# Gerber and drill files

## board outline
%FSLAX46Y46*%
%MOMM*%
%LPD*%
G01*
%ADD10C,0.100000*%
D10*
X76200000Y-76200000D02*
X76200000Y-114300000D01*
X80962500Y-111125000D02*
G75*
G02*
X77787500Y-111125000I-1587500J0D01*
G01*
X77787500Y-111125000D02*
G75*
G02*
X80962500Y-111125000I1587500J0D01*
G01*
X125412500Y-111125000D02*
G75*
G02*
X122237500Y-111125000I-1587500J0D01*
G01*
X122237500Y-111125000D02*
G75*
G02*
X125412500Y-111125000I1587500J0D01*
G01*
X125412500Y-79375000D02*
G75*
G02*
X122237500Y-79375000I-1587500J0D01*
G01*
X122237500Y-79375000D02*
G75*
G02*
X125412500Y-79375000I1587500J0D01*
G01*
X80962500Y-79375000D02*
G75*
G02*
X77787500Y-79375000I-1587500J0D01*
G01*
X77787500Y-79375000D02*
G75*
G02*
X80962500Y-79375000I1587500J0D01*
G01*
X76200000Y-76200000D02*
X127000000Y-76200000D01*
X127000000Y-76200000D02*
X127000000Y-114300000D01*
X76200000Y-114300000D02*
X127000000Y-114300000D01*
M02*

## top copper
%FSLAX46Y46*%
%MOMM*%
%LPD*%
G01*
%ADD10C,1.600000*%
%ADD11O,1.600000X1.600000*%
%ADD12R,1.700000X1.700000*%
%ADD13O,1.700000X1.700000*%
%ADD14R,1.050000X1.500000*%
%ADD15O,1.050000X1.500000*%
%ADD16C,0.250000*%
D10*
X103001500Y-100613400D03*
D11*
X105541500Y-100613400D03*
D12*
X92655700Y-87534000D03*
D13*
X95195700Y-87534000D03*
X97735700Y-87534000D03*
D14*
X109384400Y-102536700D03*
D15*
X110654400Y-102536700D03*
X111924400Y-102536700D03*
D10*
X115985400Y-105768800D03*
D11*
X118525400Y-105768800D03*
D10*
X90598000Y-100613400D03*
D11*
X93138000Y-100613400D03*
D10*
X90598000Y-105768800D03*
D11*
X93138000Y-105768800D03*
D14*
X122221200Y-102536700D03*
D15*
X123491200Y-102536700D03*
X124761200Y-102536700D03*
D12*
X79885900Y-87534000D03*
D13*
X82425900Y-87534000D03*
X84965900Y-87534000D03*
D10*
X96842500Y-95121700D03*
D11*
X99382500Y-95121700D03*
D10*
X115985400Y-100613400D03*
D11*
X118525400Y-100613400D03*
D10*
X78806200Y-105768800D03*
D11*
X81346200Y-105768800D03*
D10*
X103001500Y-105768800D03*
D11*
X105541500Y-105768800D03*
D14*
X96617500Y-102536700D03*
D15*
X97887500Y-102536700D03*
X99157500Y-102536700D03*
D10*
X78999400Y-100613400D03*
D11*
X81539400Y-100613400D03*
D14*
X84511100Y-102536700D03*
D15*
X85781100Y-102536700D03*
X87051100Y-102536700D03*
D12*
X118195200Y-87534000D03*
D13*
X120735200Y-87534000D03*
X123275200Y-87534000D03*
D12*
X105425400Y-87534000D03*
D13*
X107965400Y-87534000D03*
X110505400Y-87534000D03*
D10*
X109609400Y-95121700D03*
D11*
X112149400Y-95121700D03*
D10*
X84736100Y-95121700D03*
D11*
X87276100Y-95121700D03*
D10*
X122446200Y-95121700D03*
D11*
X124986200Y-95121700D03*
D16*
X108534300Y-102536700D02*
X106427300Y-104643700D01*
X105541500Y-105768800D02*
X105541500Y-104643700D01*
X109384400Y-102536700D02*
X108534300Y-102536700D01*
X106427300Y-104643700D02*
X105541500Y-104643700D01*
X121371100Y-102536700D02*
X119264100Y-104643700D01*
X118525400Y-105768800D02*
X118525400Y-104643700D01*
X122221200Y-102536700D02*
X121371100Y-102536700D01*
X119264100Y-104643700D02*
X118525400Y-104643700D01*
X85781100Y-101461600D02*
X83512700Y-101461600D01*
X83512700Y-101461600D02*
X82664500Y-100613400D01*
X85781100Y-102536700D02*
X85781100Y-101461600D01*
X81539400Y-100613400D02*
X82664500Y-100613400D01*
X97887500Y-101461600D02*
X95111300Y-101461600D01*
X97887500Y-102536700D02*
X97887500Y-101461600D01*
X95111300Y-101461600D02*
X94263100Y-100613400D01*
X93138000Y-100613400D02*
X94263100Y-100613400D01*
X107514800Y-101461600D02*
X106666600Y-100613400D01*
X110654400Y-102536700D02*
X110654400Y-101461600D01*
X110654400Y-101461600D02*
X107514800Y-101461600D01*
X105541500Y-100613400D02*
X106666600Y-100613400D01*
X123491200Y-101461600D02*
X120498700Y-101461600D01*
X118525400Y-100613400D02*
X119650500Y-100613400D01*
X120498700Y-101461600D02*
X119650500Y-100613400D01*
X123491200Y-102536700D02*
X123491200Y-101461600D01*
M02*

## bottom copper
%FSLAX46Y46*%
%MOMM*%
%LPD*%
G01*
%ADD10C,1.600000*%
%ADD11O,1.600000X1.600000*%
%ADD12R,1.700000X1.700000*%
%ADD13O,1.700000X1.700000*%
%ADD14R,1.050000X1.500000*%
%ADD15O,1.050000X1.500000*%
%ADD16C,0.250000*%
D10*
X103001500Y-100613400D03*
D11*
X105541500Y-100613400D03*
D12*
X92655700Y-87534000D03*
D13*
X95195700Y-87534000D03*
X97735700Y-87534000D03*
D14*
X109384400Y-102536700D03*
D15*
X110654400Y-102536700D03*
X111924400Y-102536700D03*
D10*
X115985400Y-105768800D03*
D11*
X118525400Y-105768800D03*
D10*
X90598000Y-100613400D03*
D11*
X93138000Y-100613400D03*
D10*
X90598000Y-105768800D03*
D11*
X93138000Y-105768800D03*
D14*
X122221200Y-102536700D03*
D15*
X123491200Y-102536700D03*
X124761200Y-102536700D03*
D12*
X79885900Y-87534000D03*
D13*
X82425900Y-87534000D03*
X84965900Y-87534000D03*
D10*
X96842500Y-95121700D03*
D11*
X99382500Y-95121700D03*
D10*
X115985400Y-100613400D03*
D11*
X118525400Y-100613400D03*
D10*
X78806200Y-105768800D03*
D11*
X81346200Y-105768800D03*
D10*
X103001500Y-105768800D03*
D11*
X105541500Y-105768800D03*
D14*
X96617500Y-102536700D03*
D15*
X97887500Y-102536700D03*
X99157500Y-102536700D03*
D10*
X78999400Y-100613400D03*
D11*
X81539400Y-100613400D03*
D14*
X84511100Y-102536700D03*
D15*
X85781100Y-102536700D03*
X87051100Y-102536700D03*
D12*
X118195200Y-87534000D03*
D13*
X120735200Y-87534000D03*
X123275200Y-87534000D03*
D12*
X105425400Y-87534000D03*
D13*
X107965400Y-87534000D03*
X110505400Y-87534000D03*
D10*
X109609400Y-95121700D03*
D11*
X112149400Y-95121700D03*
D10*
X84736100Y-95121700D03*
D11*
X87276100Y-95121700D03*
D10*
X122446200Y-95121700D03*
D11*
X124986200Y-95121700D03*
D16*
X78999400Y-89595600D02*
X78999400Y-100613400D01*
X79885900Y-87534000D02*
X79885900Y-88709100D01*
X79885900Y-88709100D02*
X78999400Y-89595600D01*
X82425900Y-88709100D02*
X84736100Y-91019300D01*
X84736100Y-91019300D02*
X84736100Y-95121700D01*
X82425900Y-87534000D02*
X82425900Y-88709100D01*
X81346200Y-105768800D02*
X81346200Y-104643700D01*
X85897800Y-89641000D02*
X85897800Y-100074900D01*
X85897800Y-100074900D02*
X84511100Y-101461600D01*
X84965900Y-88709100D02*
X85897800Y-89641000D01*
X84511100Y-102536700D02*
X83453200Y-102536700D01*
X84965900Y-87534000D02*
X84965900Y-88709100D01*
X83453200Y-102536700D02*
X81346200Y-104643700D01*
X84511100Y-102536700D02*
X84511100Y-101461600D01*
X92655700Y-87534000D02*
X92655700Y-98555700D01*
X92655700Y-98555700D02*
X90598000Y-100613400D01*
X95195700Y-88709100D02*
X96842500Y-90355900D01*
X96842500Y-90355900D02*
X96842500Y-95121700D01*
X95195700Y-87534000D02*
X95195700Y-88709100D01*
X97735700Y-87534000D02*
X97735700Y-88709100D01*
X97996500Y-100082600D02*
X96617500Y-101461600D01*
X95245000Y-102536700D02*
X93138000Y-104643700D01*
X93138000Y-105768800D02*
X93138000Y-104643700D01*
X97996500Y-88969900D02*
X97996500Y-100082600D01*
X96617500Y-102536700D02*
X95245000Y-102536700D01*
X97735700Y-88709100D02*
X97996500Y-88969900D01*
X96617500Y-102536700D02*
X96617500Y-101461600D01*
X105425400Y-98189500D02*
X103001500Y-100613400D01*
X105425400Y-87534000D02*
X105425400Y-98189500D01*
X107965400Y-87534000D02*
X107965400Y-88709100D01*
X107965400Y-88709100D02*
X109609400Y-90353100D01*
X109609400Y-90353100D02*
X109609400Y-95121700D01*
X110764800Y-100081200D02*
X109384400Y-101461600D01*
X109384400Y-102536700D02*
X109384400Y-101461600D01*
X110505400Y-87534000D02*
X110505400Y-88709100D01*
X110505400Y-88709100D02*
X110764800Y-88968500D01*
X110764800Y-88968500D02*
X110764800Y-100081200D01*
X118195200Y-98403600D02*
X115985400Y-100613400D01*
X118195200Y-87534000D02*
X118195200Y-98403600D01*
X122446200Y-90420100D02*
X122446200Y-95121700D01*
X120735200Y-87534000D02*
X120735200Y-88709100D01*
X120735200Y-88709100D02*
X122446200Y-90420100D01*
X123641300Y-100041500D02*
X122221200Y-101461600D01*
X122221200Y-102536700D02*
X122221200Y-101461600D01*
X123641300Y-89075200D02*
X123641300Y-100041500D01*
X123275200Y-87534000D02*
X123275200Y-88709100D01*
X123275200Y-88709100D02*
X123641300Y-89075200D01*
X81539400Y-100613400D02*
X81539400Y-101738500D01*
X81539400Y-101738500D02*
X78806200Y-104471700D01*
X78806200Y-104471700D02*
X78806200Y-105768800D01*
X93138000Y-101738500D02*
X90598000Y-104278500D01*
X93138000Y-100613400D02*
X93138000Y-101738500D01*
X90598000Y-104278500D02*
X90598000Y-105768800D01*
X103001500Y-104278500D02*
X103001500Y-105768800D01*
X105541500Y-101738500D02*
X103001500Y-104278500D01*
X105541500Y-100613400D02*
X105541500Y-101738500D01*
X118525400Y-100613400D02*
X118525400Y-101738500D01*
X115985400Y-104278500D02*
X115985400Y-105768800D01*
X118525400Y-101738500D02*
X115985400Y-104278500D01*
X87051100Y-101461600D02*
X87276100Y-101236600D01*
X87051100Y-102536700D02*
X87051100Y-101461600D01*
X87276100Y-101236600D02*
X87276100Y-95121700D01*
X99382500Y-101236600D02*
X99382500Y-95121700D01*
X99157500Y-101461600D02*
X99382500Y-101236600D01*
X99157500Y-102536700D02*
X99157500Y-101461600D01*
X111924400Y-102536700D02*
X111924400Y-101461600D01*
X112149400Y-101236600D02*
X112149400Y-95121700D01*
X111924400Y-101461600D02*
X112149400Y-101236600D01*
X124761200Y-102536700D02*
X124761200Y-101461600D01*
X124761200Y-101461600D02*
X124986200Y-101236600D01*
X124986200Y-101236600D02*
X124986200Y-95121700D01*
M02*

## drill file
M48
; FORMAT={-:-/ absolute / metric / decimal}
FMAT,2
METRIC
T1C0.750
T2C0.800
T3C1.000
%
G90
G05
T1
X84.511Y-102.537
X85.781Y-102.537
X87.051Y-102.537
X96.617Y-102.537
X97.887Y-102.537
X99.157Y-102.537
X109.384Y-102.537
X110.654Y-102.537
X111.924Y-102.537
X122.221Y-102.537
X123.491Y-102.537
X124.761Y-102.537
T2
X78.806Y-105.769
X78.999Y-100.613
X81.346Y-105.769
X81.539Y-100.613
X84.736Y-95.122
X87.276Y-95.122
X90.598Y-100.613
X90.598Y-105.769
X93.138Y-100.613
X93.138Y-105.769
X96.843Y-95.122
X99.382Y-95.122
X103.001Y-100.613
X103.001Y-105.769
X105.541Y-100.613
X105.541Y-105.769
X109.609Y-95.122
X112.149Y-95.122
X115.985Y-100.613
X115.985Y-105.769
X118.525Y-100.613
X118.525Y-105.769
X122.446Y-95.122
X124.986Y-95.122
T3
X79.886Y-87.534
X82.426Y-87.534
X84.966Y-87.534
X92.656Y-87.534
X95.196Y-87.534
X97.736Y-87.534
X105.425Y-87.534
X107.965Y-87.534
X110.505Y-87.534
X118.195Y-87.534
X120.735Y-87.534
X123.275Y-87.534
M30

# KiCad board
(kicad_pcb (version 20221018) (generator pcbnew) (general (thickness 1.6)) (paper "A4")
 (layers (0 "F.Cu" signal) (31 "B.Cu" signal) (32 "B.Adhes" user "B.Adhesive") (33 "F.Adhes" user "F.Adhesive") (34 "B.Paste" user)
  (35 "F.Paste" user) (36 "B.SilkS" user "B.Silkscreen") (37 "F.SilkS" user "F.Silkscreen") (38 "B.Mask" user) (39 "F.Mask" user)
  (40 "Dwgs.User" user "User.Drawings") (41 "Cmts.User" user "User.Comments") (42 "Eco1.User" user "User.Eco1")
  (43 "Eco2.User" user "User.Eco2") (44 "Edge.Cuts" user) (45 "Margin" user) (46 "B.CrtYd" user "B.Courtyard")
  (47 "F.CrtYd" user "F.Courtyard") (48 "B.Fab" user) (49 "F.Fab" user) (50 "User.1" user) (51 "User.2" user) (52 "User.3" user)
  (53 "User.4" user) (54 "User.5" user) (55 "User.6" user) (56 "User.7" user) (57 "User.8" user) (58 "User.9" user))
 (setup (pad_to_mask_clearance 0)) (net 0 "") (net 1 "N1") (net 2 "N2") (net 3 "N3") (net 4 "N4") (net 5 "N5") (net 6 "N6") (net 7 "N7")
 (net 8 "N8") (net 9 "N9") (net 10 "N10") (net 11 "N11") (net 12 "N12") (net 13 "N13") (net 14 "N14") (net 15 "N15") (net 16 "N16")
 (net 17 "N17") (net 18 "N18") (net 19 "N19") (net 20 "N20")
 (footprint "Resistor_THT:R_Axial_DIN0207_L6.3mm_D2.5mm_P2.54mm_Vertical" (layer "F.Cu") (at 103.0015 100.6134)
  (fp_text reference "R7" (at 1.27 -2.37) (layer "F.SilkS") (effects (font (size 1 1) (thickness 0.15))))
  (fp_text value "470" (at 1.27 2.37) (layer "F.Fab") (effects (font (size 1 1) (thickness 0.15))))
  (pad "1" thru_hole circle (at 0 0) (size 1.6 1.6) (drill 0.8) (layers "*.Cu" "*.Mask") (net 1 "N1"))
  (pad "2" thru_hole oval (at 2.54 0) (size 1.6 1.6) (drill 0.8) (layers "*.Cu" "*.Mask") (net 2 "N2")))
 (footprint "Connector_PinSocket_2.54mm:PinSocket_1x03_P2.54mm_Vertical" (layer "F.Cu") (at 92.6557 87.534 90)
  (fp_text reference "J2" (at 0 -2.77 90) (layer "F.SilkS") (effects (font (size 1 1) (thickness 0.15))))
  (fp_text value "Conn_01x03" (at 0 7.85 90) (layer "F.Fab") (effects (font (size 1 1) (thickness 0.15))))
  (pad "1" thru_hole rect (at 0 0 90) (size 1.7 1.7) (drill 1) (layers "*.Cu" "*.Mask") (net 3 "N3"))
  (pad "2" thru_hole oval (at 0 2.54 90) (size 1.7 1.7) (drill 1) (layers "*.Cu" "*.Mask") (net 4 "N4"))
  (pad "3" thru_hole oval (at 0 5.08 90) (size 1.7 1.7) (drill 1) (layers "*.Cu" "*.Mask") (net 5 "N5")))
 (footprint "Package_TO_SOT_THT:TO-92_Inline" (layer "F.Cu") (at 109.3844 102.5367)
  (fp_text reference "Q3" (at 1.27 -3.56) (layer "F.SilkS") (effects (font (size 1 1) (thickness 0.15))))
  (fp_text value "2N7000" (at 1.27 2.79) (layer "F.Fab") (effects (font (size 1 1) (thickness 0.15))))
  (pad "1" thru_hole rect (at 0 0) (size 1.05 1.5) (drill 0.75) (layers "*.Cu" "*.Mask") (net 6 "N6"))
  (pad "2" thru_hole oval (at 1.27 0) (size 1.05 1.5) (drill 0.75) (layers "*.Cu" "*.Mask") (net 2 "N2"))
  (pad "3" thru_hole oval (at 2.54 0) (size 1.05 1.5) (drill 0.75) (layers "*.Cu" "*.Mask") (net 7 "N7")))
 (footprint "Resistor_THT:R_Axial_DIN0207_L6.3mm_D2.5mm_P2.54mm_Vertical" (layer "F.Cu") (at 115.9854 105.7688)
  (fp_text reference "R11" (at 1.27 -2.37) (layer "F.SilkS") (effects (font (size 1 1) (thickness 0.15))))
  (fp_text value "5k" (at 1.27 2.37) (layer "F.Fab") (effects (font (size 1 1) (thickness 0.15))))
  (pad "1" thru_hole circle (at 0 0) (size 1.6 1.6) (drill 0.8) (layers "*.Cu" "*.Mask") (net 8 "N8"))
  (pad "2" thru_hole oval (at 2.54 0) (size 1.6 1.6) (drill 0.8) (layers "*.Cu" "*.Mask") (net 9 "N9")))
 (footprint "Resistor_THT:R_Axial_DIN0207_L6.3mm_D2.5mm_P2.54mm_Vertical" (layer "F.Cu") (at 90.598 100.6134)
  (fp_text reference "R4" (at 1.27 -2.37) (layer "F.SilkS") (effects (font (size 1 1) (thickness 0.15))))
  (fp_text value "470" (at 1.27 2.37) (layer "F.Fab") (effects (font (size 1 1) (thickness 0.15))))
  (pad "1" thru_hole circle (at 0 0) (size 1.6 1.6) (drill 0.8) (layers "*.Cu" "*.Mask") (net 3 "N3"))
  (pad "2" thru_hole oval (at 2.54 0) (size 1.6 1.6) (drill 0.8) (layers "*.Cu" "*.Mask") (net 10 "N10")))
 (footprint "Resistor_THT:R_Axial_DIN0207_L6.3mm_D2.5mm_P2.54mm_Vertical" (layer "F.Cu") (at 90.598 105.7688)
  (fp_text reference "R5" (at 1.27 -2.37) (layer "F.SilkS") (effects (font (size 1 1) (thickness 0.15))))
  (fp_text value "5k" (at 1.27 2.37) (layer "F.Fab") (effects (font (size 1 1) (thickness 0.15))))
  (pad "1" thru_hole circle (at 0 0) (size 1.6 1.6) (drill 0.8) (layers "*.Cu" "*.Mask") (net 10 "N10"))
  (pad "2" thru_hole oval (at 2.54 0) (size 1.6 1.6) (drill 0.8) (layers "*.Cu" "*.Mask") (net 5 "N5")))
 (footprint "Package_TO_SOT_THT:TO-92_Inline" (layer "F.Cu") (at 122.2212 102.5367)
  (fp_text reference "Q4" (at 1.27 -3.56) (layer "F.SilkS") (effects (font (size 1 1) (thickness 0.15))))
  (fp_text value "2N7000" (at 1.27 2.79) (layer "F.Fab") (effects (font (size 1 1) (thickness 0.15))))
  (pad "1" thru_hole rect (at 0 0) (size 1.05 1.5) (drill 0.75) (layers "*.Cu" "*.Mask") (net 9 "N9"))
  (pad "2" thru_hole oval (at 1.27 0) (size 1.05 1.5) (drill 0.75) (layers "*.Cu" "*.Mask") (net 8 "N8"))
  (pad "3" thru_hole oval (at 2.54 0) (size 1.05 1.5) (drill 0.75) (layers "*.Cu" "*.Mask") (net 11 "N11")))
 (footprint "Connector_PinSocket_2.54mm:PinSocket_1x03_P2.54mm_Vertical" (layer "F.Cu") (at 79.8859 87.534 90)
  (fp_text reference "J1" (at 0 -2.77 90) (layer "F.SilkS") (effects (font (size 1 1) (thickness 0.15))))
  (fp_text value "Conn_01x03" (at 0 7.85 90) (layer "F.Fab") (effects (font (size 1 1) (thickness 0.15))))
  (pad "1" thru_hole rect (at 0 0 90) (size 1.7 1.7) (drill 1) (layers "*.Cu" "*.Mask") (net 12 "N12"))
  (pad "2" thru_hole oval (at 0 2.54 90) (size 1.7 1.7) (drill 1) (layers "*.Cu" "*.Mask") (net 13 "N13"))
  (pad "3" thru_hole oval (at 0 5.08 90) (size 1.7 1.7) (drill 1) (layers "*.Cu" "*.Mask") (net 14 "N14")))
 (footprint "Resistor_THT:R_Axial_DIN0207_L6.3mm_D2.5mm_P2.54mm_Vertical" (layer "F.Cu") (at 96.8425 95.1217)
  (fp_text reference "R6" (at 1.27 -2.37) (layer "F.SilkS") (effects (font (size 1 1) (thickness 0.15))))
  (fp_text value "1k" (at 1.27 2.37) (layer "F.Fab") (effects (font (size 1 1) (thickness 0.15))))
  (pad "1" thru_hole circle (at 0 0) (size 1.6 1.6) (drill 0.8) (layers "*.Cu" "*.Mask") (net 4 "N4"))
  (pad "2" thru_hole oval (at 2.54 0) (size 1.6 1.6) (drill 0.8) (layers "*.Cu" "*.Mask") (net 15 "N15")))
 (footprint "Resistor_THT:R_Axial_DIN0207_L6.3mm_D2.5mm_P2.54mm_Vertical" (layer "F.Cu") (at 115.9854 100.6134)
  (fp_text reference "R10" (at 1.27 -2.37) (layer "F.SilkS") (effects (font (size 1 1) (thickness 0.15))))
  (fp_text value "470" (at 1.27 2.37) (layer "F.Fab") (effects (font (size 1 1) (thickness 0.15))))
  (pad "1" thru_hole circle (at 0 0) (size 1.6 1.6) (drill 0.8) (layers "*.Cu" "*.Mask") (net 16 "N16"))
  (pad "2" thru_hole oval (at 2.54 0) (size 1.6 1.6) (drill 0.8) (layers "*.Cu" "*.Mask") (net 8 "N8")))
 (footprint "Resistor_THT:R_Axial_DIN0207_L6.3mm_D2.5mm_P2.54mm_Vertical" (layer "F.Cu") (at 78.8062 105.7688)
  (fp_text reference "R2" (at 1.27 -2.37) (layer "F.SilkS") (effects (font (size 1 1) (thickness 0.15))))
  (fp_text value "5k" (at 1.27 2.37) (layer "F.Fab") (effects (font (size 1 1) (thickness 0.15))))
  (pad "1" thru_hole circle (at 0 0) (size 1.6 1.6) (drill 0.8) (layers "*.Cu" "*.Mask") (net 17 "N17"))
  (pad "2" thru_hole oval (at 2.54 0) (size 1.6 1.6) (drill 0.8) (layers "*.Cu" "*.Mask") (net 14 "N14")))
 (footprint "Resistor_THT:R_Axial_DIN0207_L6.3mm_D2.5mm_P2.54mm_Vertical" (layer "F.Cu") (at 103.0015 105.7688)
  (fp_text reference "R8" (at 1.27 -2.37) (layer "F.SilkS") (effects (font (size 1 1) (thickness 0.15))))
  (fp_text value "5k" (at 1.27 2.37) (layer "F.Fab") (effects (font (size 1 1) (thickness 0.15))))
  (pad "1" thru_hole circle (at 0 0) (size 1.6 1.6) (drill 0.8) (layers "*.Cu" "*.Mask") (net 2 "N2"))
  (pad "2" thru_hole oval (at 2.54 0) (size 1.6 1.6) (drill 0.8) (layers "*.Cu" "*.Mask") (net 6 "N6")))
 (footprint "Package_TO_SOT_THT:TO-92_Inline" (layer "F.Cu") (at 96.6175 102.5367)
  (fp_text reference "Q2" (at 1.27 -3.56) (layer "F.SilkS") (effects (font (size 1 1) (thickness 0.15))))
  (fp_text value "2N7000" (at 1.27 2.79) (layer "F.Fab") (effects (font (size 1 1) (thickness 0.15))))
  (pad "1" thru_hole rect (at 0 0) (size 1.05 1.5) (drill 0.75) (layers "*.Cu" "*.Mask") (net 5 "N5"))
  (pad "2" thru_hole oval (at 1.27 0) (size 1.05 1.5) (drill 0.75) (layers "*.Cu" "*.Mask") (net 10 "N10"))
  (pad "3" thru_hole oval (at 2.54 0) (size 1.05 1.5) (drill 0.75) (layers "*.Cu" "*.Mask") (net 15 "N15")))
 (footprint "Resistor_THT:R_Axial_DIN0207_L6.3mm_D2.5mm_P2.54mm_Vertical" (layer "F.Cu") (at 78.9994 100.6134)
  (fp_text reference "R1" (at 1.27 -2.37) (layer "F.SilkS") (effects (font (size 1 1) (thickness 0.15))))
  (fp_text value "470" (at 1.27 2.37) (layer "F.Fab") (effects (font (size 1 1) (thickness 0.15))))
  (pad "1" thru_hole circle (at 0 0) (size 1.6 1.6) (drill 0.8) (layers "*.Cu" "*.Mask") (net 12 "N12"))
  (pad "2" thru_hole oval (at 2.54 0) (size 1.6 1.6) (drill 0.8) (layers "*.Cu" "*.Mask") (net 17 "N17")))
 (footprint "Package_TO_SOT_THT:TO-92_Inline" (layer "F.Cu") (at 84.5111 102.5367)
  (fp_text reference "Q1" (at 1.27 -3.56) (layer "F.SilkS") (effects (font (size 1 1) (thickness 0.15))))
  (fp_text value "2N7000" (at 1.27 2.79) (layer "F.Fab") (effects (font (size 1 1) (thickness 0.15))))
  (pad "1" thru_hole rect (at 0 0) (size 1.05 1.5) (drill 0.75) (layers "*.Cu" "*.Mask") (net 14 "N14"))
  (pad "2" thru_hole oval (at 1.27 0) (size 1.05 1.5) (drill 0.75) (layers "*.Cu" "*.Mask") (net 17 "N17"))
  (pad "3" thru_hole oval (at 2.54 0) (size 1.05 1.5) (drill 0.75) (layers "*.Cu" "*.Mask") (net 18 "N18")))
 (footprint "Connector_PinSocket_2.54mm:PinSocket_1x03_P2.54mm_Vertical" (layer "F.Cu") (at 118.1952 87.534 90)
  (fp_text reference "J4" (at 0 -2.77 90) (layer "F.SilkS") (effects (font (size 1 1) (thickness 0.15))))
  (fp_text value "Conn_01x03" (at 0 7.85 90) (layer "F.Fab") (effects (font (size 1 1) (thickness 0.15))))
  (pad "1" thru_hole rect (at 0 0 90) (size 1.7 1.7) (drill 1) (layers "*.Cu" "*.Mask") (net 16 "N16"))
  (pad "2" thru_hole oval (at 0 2.54 90) (size 1.7 1.7) (drill 1) (layers "*.Cu" "*.Mask") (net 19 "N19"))
  (pad "3" thru_hole oval (at 0 5.08 90) (size 1.7 1.7) (drill 1) (layers "*.Cu" "*.Mask") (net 9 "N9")))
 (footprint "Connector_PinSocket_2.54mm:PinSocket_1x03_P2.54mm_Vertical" (layer "F.Cu") (at 105.4254 87.534 90)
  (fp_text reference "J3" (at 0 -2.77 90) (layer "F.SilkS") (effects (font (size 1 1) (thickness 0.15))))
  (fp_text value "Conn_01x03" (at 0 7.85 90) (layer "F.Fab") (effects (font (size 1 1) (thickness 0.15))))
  (pad "1" thru_hole rect (at 0 0 90) (size 1.7 1.7) (drill 1) (layers "*.Cu" "*.Mask") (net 1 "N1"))
  (pad "2" thru_hole oval (at 0 2.54 90) (size 1.7 1.7) (drill 1) (layers "*.Cu" "*.Mask") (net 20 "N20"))
  (pad "3" thru_hole oval (at 0 5.08 90) (size 1.7 1.7) (drill 1) (layers "*.Cu" "*.Mask") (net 6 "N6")))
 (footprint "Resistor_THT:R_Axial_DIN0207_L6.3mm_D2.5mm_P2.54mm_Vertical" (layer "F.Cu") (at 109.6094 95.1217)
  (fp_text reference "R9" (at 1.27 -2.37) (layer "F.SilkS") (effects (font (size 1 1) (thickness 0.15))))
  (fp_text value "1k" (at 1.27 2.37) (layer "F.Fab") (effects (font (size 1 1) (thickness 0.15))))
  (pad "1" thru_hole circle (at 0 0) (size 1.6 1.6) (drill 0.8) (layers "*.Cu" "*.Mask") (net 20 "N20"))
  (pad "2" thru_hole oval (at 2.54 0) (size 1.6 1.6) (drill 0.8) (layers "*.Cu" "*.Mask") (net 7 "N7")))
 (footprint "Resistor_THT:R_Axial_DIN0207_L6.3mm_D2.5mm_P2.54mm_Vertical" (layer "F.Cu") (at 84.7361 95.1217)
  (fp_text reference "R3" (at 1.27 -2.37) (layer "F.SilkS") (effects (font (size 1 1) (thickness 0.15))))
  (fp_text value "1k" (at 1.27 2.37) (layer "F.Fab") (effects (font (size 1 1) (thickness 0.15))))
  (pad "1" thru_hole circle (at 0 0) (size 1.6 1.6) (drill 0.8) (layers "*.Cu" "*.Mask") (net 13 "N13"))
  (pad "2" thru_hole oval (at 2.54 0) (size 1.6 1.6) (drill 0.8) (layers "*.Cu" "*.Mask") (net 18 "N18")))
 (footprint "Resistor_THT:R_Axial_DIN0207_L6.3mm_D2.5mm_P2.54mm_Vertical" (layer "F.Cu") (at 122.4462 95.1217)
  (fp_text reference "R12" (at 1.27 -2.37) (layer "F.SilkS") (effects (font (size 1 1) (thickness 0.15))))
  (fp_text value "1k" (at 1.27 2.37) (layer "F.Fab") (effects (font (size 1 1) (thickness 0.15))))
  (pad "1" thru_hole circle (at 0 0) (size 1.6 1.6) (drill 0.8) (layers "*.Cu" "*.Mask") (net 19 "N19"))
  (pad "2" thru_hole oval (at 2.54 0) (size 1.6 1.6) (drill 0.8) (layers "*.Cu" "*.Mask") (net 11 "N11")))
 (gr_line (start 76.2 76.2) (end 76.2 114.3) (stroke (width 0.1) (type default)) (layer "Edge.Cuts"))
 (gr_circle (center 79.375 111.125) (end 80.9625 111.125) (stroke (width 0.1) (type default)) (fill none) (layer "Edge.Cuts"))
 (gr_circle (center 123.825 111.125) (end 125.4125 111.125) (stroke (width 0.1) (type default)) (fill none) (layer "Edge.Cuts"))
 (gr_circle (center 123.825 79.375) (end 125.4125 79.375) (stroke (width 0.1) (type default)) (fill none) (layer "Edge.Cuts"))
 (gr_circle (center 79.375 79.375) (end 80.9625 79.375) (stroke (width 0.1) (type default)) (fill none) (layer "Edge.Cuts"))
 (gr_line (start 76.2 76.2) (end 127 76.2) (stroke (width 0.1) (type default)) (layer "Edge.Cuts"))
 (gr_line (start 127 76.2) (end 127 114.3) (stroke (width 0.1) (type default)) (layer "Edge.Cuts"))
 (gr_line (start 76.2 114.3) (end 127 114.3) (stroke (width 0.1) (type default)) (layer "Edge.Cuts"))
 (segment (start 78.9994 89.5956) (end 78.9994 100.6134) (width 0.25) (layer "B.Cu") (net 12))
 (segment (start 79.8859 87.534) (end 79.8859 88.7091) (width 0.25) (layer "B.Cu") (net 12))
 (segment (start 79.8859 88.7091) (end 78.9994 89.5956) (width 0.25) (layer "B.Cu") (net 12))
 (segment (start 82.4259 88.7091) (end 84.7361 91.0193) (width 0.25) (layer "B.Cu") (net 13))
 (segment (start 84.7361 91.0193) (end 84.7361 95.1217) (width 0.25) (layer "B.Cu") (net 13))
 (segment (start 82.4259 87.534) (end 82.4259 88.7091) (width 0.25) (layer "B.Cu") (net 13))
 (segment (start 81.3462 105.7688) (end 81.3462 104.6437) (width 0.25) (layer "B.Cu") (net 14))
 (segment (start 85.8978 89.641) (end 85.8978 100.0749) (width 0.25) (layer "B.Cu") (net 14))
 (segment (start 85.8978 100.0749) (end 84.5111 101.4616) (width 0.25) (layer "B.Cu") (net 14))
 (segment (start 84.9659 88.7091) (end 85.8978 89.641) (width 0.25) (layer "B.Cu") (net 14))
 (segment (start 84.5111 102.5367) (end 83.4532 102.5367) (width 0.25) (layer "B.Cu") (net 14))
 (segment (start 84.9659 87.534) (end 84.9659 88.7091) (width 0.25) (layer "B.Cu") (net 14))
 (segment (start 83.4532 102.5367) (end 81.3462 104.6437) (width 0.25) (layer "B.Cu") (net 14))
 (segment (start 84.5111 102.5367) (end 84.5111 101.4616) (width 0.25) (layer "B.Cu") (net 14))
 (segment (start 92.6557 87.534) (end 92.6557 98.5557) (width 0.25) (layer "B.Cu") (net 3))
 (segment (start 92.6557 98.5557) (end 90.598 100.6134) (width 0.25) (layer "B.Cu") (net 3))
 (segment (start 95.1957 88.7091) (end 96.8425 90.3559) (width 0.25) (layer "B.Cu") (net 4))
 (segment (start 96.8425 90.3559) (end 96.8425 95.1217) (width 0.25) (layer "B.Cu") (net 4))
 (segment (start 95.1957 87.534) (end 95.1957 88.7091) (width 0.25) (layer "B.Cu") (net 4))
 (segment (start 97.7357 87.534) (end 97.7357 88.7091) (width 0.25) (layer "B.Cu") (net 5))
 (segment (start 97.9965 100.0826) (end 96.6175 101.4616) (width 0.25) (layer "B.Cu") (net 5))
 (segment (start 95.245 102.5367) (end 93.138 104.6437) (width 0.25) (layer "B.Cu") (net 5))
 (segment (start 93.138 105.7688) (end 93.138 104.6437) (width 0.25) (layer "B.Cu") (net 5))
 (segment (start 97.9965 88.9699) (end 97.9965 100.0826) (width 0.25) (layer "B.Cu") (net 5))
 (segment (start 96.6175 102.5367) (end 95.245 102.5367) (width 0.25) (layer "B.Cu") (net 5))
 (segment (start 97.7357 88.7091) (end 97.9965 88.9699) (width 0.25) (layer "B.Cu") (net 5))
 (segment (start 96.6175 102.5367) (end 96.6175 101.4616) (width 0.25) (layer "B.Cu") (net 5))
 (segment (start 105.4254 98.1895) (end 103.0015 100.6134) (width 0.25) (layer "B.Cu") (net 1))
 (segment (start 105.4254 87.534) (end 105.4254 98.1895) (width 0.25) (layer "B.Cu") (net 1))
 (segment (start 107.9654 87.534) (end 107.9654 88.7091) (width 0.25) (layer "B.Cu") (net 20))
 (segment (start 107.9654 88.7091) (end 109.6094 90.3531) (width 0.25) (layer "B.Cu") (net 20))
 (segment (start 109.6094 90.3531) (end 109.6094 95.1217) (width 0.25) (layer "B.Cu") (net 20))
 (segment (start 108.5343 102.5367) (end 106.4273 104.6437) (width 0.25) (layer "F.Cu") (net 6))
 (segment (start 105.5415 105.7688) (end 105.5415 104.6437) (width 0.25) (layer "F.Cu") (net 6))
 (segment (start 109.3844 102.5367) (end 108.5343 102.5367) (width 0.25) (layer "F.Cu") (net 6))
 (segment (start 106.4273 104.6437) (end 105.5415 104.6437) (width 0.25) (layer "F.Cu") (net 6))
 (segment (start 110.7648 100.0812) (end 109.3844 101.4616) (width 0.25) (layer "B.Cu") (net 6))
 (segment (start 109.3844 102.5367) (end 109.3844 101.4616) (width 0.25) (layer "B.Cu") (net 6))
 (segment (start 110.5054 87.534) (end 110.5054 88.7091) (width 0.25) (layer "B.Cu") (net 6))
 (segment (start 110.5054 88.7091) (end 110.7648 88.9685) (width 0.25) (layer "B.Cu") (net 6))
 (segment (start 110.7648 88.9685) (end 110.7648 100.0812) (width 0.25) (layer "B.Cu") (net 6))
 (segment (start 118.1952 98.4036) (end 115.9854 100.6134) (width 0.25) (layer "B.Cu") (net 16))
 (segment (start 118.1952 87.534) (end 118.1952 98.4036) (width 0.25) (layer "B.Cu") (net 16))
 (segment (start 122.4462 90.4201) (end 122.4462 95.1217) (width 0.25) (layer "B.Cu") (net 19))
 (segment (start 120.7352 87.534) (end 120.7352 88.7091) (width 0.25) (layer "B.Cu") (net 19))
 (segment (start 120.7352 88.7091) (end 122.4462 90.4201) (width 0.25) (layer "B.Cu") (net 19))
 (segment (start 121.3711 102.5367) (end 119.2641 104.6437) (width 0.25) (layer "F.Cu") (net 9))
 (segment (start 118.5254 105.7688) (end 118.5254 104.6437) (width 0.25) (layer "F.Cu") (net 9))
 (segment (start 122.2212 102.5367) (end 121.3711 102.5367) (width 0.25) (layer "F.Cu") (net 9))
 (segment (start 119.2641 104.6437) (end 118.5254 104.6437) (width 0.25) (layer "F.Cu") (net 9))
 (segment (start 123.6413 100.0415) (end 122.2212 101.4616) (width 0.25) (layer "B.Cu") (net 9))
 (segment (start 122.2212 102.5367) (end 122.2212 101.4616) (width 0.25) (layer "B.Cu") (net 9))
 (segment (start 123.6413 89.0752) (end 123.6413 100.0415) (width 0.25) (layer "B.Cu") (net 9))
 (segment (start 123.2752 87.534) (end 123.2752 88.7091) (width 0.25) (layer "B.Cu") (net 9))
 (segment (start 123.2752 88.7091) (end 123.6413 89.0752) (width 0.25) (layer "B.Cu") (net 9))
 (segment (start 85.7811 101.4616) (end 83.5127 101.4616) (width 0.25) (layer "F.Cu") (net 17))
 (segment (start 83.5127 101.4616) (end 82.6645 100.6134) (width 0.25) (layer "F.Cu") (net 17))
 (segment (start 85.7811 102.5367) (end 85.7811 101.4616) (width 0.25) (layer "F.Cu") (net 17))
 (segment (start 81.5394 100.6134) (end 82.6645 100.6134) (width 0.25) (layer "F.Cu") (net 17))
 (segment (start 81.5394 100.6134) (end 81.5394 101.7385) (width 0.25) (layer "B.Cu") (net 17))
 (segment (start 81.5394 101.7385) (end 78.8062 104.4717) (width 0.25) (layer "B.Cu") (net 17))
 (segment (start 78.8062 104.4717) (end 78.8062 105.7688) (width 0.25) (layer "B.Cu") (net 17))
 (segment (start 97.8875 101.4616) (end 95.1113 101.4616) (width 0.25) (layer "F.Cu") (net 10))
 (segment (start 97.8875 102.5367) (end 97.8875 101.4616) (width 0.25) (layer "F.Cu") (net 10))
 (segment (start 95.1113 101.4616) (end 94.2631 100.6134) (width 0.25) (layer "F.Cu") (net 10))
 (segment (start 93.138 100.6134) (end 94.2631 100.6134) (width 0.25) (layer "F.Cu") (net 10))
 (segment (start 93.138 101.7385) (end 90.598 104.2785) (width 0.25) (layer "B.Cu") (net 10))
 (segment (start 93.138 100.6134) (end 93.138 101.7385) (width 0.25) (layer "B.Cu") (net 10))
 (segment (start 90.598 104.2785) (end 90.598 105.7688) (width 0.25) (layer "B.Cu") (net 10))
 (segment (start 107.5148 101.4616) (end 106.6666 100.6134) (width 0.25) (layer "F.Cu") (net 2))
 (segment (start 110.6544 102.5367) (end 110.6544 101.4616) (width 0.25) (layer "F.Cu") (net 2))
 (segment (start 110.6544 101.4616) (end 107.5148 101.4616) (width 0.25) (layer "F.Cu") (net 2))
 (segment (start 105.5415 100.6134) (end 106.6666 100.6134) (width 0.25) (layer "F.Cu") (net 2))
 (segment (start 103.0015 104.2785) (end 103.0015 105.7688) (width 0.25) (layer "B.Cu") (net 2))
 (segment (start 105.5415 101.7385) (end 103.0015 104.2785) (width 0.25) (layer "B.Cu") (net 2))
 (segment (start 105.5415 100.6134) (end 105.5415 101.7385) (width 0.25) (layer "B.Cu") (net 2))
 (segment (start 123.4912 101.4616) (end 120.4987 101.4616) (width 0.25) (layer "F.Cu") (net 8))
 (segment (start 118.5254 100.6134) (end 119.6505 100.6134) (width 0.25) (layer "F.Cu") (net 8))
 (segment (start 120.4987 101.4616) (end 119.6505 100.6134) (width 0.25) (layer "F.Cu") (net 8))
 (segment (start 123.4912 102.5367) (end 123.4912 101.4616) (width 0.25) (layer "F.Cu") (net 8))
 (segment (start 118.5254 100.6134) (end 118.5254 101.7385) (width 0.25) (layer "B.Cu") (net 8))
 (segment (start 115.9854 104.2785) (end 115.9854 105.7688) (width 0.25) (layer "B.Cu") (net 8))
 (segment (start 118.5254 101.7385) (end 115.9854 104.2785) (width 0.25) (layer "B.Cu") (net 8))
 (segment (start 87.0511 101.4616) (end 87.2761 101.2366) (width 0.25) (layer "B.Cu") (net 18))
 (segment (start 87.0511 102.5367) (end 87.0511 101.4616) (width 0.25) (layer "B.Cu") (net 18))
 (segment (start 87.2761 101.2366) (end 87.2761 95.1217) (width 0.25) (layer "B.Cu") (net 18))
 (segment (start 99.3825 101.2366) (end 99.3825 95.1217) (width 0.25) (layer "B.Cu") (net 15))
 (segment (start 99.1575 101.4616) (end 99.3825 101.2366) (width 0.25) (layer "B.Cu") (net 15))
 (segment (start 99.1575 102.5367) (end 99.1575 101.4616) (width 0.25) (layer "B.Cu") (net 15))
 (segment (start 111.9244 102.5367) (end 111.9244 101.4616) (width 0.25) (layer "B.Cu") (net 7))
 (segment (start 112.1494 101.2366) (end 112.1494 95.1217) (width 0.25) (layer "B.Cu") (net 7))
 (segment (start 111.9244 101.4616) (end 112.1494 101.2366) (width 0.25) (layer "B.Cu") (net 7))
 (segment (start 124.7612 102.5367) (end 124.7612 101.4616) (width 0.25) (layer "B.Cu") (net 11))
 (segment (start 124.7612 101.4616) (end 124.9862 101.2366) (width 0.25) (layer "B.Cu") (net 11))
 (segment (start 124.9862 101.2366) (end 124.9862 95.1217) (width 0.25) (layer "B.Cu") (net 11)))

